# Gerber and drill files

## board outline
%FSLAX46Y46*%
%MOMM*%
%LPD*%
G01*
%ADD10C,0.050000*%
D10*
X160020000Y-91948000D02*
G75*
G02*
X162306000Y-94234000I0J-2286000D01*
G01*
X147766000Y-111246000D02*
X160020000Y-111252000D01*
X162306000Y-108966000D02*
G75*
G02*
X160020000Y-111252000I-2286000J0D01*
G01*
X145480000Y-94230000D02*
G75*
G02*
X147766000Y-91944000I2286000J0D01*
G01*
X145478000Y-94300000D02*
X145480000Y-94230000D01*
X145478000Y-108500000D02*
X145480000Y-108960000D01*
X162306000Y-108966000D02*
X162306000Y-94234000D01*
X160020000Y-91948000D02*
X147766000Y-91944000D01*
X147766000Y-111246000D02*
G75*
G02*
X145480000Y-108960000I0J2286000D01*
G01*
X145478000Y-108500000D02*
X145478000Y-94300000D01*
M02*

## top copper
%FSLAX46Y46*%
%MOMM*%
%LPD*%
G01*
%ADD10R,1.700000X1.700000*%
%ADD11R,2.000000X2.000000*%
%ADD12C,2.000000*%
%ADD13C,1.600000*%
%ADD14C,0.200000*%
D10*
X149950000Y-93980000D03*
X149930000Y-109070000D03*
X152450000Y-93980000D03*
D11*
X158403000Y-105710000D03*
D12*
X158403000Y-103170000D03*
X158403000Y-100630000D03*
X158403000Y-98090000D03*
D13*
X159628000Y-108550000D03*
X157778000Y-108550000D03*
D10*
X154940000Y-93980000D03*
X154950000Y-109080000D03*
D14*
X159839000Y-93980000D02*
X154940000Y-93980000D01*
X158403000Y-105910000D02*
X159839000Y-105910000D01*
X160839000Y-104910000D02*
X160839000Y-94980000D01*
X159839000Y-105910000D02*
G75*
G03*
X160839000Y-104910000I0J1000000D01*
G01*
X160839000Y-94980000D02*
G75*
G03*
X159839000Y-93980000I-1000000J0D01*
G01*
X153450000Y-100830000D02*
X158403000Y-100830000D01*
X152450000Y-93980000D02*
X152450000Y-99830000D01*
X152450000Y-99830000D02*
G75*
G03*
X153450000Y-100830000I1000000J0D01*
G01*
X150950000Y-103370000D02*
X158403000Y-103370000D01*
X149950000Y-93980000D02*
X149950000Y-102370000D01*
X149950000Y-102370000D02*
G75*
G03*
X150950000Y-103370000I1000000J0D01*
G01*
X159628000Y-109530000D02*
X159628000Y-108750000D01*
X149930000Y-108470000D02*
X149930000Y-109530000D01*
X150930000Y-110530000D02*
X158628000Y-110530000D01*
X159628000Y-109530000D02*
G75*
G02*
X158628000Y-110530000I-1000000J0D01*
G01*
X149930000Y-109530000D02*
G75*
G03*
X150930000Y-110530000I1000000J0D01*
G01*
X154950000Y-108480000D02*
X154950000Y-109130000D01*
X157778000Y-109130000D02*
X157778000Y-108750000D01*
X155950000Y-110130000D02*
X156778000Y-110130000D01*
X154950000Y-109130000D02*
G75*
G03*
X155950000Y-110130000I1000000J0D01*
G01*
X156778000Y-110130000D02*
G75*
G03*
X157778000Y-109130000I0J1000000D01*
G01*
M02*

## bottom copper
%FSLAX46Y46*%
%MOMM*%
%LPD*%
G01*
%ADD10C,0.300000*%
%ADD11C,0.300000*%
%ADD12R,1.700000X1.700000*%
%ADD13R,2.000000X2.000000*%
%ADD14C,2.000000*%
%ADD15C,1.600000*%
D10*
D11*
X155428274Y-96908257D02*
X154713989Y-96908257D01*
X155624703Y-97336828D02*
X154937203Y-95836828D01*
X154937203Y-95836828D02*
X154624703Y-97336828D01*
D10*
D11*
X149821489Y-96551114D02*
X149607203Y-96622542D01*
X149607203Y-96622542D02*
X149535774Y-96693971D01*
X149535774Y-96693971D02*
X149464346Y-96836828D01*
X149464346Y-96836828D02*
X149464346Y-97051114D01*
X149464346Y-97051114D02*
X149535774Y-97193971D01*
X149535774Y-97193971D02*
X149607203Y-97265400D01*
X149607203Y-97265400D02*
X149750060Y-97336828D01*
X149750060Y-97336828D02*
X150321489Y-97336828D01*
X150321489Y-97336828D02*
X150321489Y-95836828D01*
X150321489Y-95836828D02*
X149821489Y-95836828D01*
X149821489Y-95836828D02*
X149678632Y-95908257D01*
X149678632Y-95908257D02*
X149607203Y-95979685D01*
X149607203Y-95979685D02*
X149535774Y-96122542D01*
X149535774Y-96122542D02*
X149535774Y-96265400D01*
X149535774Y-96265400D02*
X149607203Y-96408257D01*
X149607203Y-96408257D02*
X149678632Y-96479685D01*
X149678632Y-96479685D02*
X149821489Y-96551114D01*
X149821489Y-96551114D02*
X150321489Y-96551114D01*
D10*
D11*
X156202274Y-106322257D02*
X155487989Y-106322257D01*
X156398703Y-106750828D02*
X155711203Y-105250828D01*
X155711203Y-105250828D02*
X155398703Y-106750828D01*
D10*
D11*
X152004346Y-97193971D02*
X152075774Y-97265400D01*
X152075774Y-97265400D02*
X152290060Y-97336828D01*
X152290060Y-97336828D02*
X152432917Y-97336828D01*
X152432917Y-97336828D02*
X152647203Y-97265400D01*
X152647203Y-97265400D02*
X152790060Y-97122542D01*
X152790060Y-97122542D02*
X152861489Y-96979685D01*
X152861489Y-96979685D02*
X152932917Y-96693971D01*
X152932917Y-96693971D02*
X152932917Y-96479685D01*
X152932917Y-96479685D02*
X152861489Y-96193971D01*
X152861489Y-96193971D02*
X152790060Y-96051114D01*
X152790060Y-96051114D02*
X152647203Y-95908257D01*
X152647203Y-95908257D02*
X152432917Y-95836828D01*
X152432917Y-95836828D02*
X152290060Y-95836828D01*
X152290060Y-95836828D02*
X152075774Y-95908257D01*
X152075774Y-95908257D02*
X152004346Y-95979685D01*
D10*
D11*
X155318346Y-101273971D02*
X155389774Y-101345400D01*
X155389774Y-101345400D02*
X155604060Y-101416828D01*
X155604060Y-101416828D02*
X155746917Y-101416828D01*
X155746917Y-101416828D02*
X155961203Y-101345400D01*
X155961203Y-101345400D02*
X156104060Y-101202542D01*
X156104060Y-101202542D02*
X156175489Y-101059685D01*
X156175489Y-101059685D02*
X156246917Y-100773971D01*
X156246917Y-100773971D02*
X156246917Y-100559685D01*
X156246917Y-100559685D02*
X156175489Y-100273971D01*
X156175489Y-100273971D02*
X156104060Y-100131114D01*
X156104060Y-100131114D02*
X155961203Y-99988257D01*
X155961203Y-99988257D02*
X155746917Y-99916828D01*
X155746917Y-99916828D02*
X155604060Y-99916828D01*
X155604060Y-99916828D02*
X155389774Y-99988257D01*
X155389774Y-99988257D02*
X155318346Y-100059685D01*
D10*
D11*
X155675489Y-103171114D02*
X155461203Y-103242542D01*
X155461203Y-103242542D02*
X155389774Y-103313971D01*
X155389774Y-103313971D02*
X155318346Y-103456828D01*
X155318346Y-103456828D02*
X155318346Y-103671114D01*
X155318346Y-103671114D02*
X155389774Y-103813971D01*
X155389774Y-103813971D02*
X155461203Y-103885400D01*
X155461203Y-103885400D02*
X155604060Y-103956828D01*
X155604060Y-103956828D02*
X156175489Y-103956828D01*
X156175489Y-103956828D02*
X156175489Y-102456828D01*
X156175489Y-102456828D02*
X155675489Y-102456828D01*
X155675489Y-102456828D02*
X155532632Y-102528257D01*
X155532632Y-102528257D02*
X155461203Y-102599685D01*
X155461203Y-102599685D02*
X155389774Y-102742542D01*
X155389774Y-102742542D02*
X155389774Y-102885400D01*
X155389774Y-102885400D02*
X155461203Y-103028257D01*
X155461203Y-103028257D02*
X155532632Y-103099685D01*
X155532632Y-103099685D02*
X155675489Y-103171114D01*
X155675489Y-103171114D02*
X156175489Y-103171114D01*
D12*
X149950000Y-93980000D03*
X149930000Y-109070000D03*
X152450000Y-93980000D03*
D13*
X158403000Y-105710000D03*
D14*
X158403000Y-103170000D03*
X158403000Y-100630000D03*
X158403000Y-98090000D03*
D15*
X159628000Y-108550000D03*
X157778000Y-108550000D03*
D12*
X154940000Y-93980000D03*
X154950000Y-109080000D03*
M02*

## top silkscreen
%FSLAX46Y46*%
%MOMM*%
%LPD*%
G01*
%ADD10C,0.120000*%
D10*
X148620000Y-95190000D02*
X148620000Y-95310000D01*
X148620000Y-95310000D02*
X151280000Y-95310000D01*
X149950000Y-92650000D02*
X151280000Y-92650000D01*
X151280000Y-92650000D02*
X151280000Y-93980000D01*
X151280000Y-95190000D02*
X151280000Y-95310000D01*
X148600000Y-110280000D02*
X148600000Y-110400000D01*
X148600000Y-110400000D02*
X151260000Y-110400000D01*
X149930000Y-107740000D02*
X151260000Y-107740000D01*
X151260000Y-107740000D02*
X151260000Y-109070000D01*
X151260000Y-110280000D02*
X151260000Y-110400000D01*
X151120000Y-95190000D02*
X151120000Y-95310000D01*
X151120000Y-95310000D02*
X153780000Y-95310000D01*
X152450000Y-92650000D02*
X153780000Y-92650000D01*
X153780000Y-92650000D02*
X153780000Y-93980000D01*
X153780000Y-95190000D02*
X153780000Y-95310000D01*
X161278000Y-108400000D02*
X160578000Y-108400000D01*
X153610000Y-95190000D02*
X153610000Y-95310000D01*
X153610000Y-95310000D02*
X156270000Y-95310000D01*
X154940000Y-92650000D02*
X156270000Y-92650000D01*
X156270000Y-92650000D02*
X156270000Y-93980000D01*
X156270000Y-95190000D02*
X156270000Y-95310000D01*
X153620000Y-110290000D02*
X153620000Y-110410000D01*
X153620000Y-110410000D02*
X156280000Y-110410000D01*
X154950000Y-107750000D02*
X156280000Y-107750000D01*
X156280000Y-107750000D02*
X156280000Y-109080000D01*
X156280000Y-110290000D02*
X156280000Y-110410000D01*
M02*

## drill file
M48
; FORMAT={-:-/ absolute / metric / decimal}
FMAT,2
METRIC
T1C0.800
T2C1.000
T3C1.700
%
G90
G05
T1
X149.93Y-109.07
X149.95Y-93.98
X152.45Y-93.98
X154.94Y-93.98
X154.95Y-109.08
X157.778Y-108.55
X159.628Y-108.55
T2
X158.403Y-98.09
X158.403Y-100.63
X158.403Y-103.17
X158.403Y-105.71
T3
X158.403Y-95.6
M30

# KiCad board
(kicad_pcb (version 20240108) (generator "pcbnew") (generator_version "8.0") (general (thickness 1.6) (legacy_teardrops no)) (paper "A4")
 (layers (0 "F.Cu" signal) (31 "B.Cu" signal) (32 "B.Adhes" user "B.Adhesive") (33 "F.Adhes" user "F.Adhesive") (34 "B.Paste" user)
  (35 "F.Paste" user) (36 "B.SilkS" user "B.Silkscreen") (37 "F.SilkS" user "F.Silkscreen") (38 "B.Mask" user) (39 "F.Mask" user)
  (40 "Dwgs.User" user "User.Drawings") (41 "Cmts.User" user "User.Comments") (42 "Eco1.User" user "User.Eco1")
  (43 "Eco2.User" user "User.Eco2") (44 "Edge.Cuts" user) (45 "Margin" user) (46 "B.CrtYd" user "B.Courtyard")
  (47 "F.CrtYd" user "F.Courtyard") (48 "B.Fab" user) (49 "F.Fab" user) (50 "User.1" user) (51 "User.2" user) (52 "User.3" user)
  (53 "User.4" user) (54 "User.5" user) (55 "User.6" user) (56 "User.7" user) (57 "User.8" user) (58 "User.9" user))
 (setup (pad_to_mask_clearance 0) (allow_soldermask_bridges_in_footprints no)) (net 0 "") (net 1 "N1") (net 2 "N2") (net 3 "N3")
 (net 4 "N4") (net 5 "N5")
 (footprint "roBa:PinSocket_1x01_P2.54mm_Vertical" (layer "F.Cu") (at 149.95 93.98)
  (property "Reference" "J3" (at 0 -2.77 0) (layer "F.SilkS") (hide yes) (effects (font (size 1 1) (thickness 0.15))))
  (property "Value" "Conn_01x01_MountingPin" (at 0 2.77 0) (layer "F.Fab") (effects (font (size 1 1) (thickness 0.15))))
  (fp_line (start -1.33 1.21) (end -1.33 1.33) (stroke (width 0.12) (type solid)) (layer "F.SilkS"))
  (fp_line (start -1.33 1.33) (end 1.33 1.33) (stroke (width 0.12) (type solid)) (layer "F.SilkS"))
  (fp_line (start 0 -1.33) (end 1.33 -1.33) (stroke (width 0.12) (type solid)) (layer "F.SilkS"))
  (fp_line (start 1.33 -1.33) (end 1.33 0) (stroke (width 0.12) (type solid)) (layer "F.SilkS"))
  (fp_line (start 1.33 1.21) (end 1.33 1.33) (stroke (width 0.12) (type solid)) (layer "F.SilkS"))
  (pad "1" thru_hole rect (at 0 0) (size 1.7 1.7) (drill 0.8) (layers "*.Cu" "*.Mask") (remove_unused_layers no) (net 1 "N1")))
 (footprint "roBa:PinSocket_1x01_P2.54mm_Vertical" (layer "F.Cu") (at 149.93 109.07)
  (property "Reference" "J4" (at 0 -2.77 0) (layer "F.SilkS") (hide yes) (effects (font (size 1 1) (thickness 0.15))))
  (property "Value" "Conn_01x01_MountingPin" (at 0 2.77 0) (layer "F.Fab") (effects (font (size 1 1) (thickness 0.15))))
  (fp_line (start -1.33 1.21) (end -1.33 1.33) (stroke (width 0.12) (type solid)) (layer "F.SilkS"))
  (fp_line (start -1.33 1.33) (end 1.33 1.33) (stroke (width 0.12) (type solid)) (layer "F.SilkS"))
  (fp_line (start 0 -1.33) (end 1.33 -1.33) (stroke (width 0.12) (type solid)) (layer "F.SilkS"))
  (fp_line (start 1.33 -1.33) (end 1.33 0) (stroke (width 0.12) (type solid)) (layer "F.SilkS"))
  (fp_line (start 1.33 1.21) (end 1.33 1.33) (stroke (width 0.12) (type solid)) (layer "F.SilkS"))
  (pad "1" thru_hole rect (at 0 0) (size 1.7 1.7) (drill 0.8) (layers "*.Cu" "*.Mask") (remove_unused_layers no) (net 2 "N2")))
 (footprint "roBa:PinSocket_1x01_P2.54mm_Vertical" (layer "F.Cu") (at 152.45 93.98)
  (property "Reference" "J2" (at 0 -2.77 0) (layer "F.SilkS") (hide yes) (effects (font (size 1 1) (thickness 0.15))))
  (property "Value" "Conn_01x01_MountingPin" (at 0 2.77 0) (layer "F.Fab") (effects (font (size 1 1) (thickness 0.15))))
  (fp_line (start -1.33 1.21) (end -1.33 1.33) (stroke (width 0.12) (type solid)) (layer "F.SilkS"))
  (fp_line (start -1.33 1.33) (end 1.33 1.33) (stroke (width 0.12) (type solid)) (layer "F.SilkS"))
  (fp_line (start 0 -1.33) (end 1.33 -1.33) (stroke (width 0.12) (type solid)) (layer "F.SilkS"))
  (fp_line (start 1.33 -1.33) (end 1.33 0) (stroke (width 0.12) (type solid)) (layer "F.SilkS"))
  (fp_line (start 1.33 1.21) (end 1.33 1.33) (stroke (width 0.12) (type solid)) (layer "F.SilkS"))
  (pad "1" thru_hole rect (at 0 0) (size 1.7 1.7) (drill 0.8) (layers "*.Cu" "*.Mask") (remove_unused_layers no) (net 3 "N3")))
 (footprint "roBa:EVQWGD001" (layer "F.Cu") (at 151.518 101.4 180)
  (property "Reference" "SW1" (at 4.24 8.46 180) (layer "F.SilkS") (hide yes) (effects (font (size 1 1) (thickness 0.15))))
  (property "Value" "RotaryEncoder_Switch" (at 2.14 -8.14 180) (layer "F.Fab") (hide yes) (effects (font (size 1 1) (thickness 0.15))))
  (fp_line (start -9.76 -7) (end -9.06 -7) (stroke (width 0.12) (type solid)) (layer "F.SilkS"))
  (fp_line (start 6.04 -7.1) (end 6.04 7.1) (stroke (width 0.05) (type solid)) (layer "Edge.Cuts"))
  (pad "" np_thru_hole circle (at -6.885 5.8 180) (size 1.7 1.7) (drill 1.7) (layers "*.Cu" "*.Mask"))
  (pad "A" thru_hole rect (at -6.885 -4.31 180) (size 2 2) (drill 1) (layers "*.Cu" "*.Mask") (remove_unused_layers no) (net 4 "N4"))
  (pad "B" thru_hole circle (at -6.885 -1.77 180) (size 2 2) (drill 1) (layers "*.Cu" "*.Mask") (remove_unused_layers no) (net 1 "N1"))
  (pad "C" thru_hole circle (at -6.885 0.77 180) (size 2 2) (drill 1) (layers "*.Cu" "*.Mask") (remove_unused_layers no) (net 3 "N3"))
  (pad "D" thru_hole circle (at -6.885 3.31 180) (size 2 2) (drill 1) (layers "*.Cu" "*.Mask") (remove_unused_layers no))
  (pad "S1" thru_hole circle (at -8.11 -7.15 180) (size 1.6 1.6) (drill 0.8) (layers "*.Cu" "*.Mask") (remove_unused_layers no) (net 2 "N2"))
  (pad "S2" thru_hole circle (at -6.26 -7.15 180) (size 1.6 1.6) (drill 0.8) (layers "*.Cu" "*.Mask") (remove_unused_layers no) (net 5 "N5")))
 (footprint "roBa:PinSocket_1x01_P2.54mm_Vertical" (layer "F.Cu") (at 154.94 93.98)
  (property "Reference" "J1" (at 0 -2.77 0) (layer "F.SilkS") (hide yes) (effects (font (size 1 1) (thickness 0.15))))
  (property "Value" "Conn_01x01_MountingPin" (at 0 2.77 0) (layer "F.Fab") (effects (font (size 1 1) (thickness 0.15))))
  (fp_line (start -1.33 1.21) (end -1.33 1.33) (stroke (width 0.12) (type solid)) (layer "F.SilkS"))
  (fp_line (start -1.33 1.33) (end 1.33 1.33) (stroke (width 0.12) (type solid)) (layer "F.SilkS"))
  (fp_line (start 0 -1.33) (end 1.33 -1.33) (stroke (width 0.12) (type solid)) (layer "F.SilkS"))
  (fp_line (start 1.33 -1.33) (end 1.33 0) (stroke (width 0.12) (type solid)) (layer "F.SilkS"))
  (fp_line (start 1.33 1.21) (end 1.33 1.33) (stroke (width 0.12) (type solid)) (layer "F.SilkS"))
  (pad "1" thru_hole rect (at 0 0) (size 1.7 1.7) (drill 0.8) (layers "*.Cu" "*.Mask") (remove_unused_layers no) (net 4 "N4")))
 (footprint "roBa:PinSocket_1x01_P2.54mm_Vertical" (layer "F.Cu") (at 154.95 109.08)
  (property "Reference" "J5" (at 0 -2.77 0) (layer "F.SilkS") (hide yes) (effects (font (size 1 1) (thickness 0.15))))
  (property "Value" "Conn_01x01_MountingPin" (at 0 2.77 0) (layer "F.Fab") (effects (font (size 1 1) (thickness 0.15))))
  (fp_line (start -1.33 1.21) (end -1.33 1.33) (stroke (width 0.12) (type solid)) (layer "F.SilkS"))
  (fp_line (start -1.33 1.33) (end 1.33 1.33) (stroke (width 0.12) (type solid)) (layer "F.SilkS"))
  (fp_line (start 0 -1.33) (end 1.33 -1.33) (stroke (width 0.12) (type solid)) (layer "F.SilkS"))
  (fp_line (start 1.33 -1.33) (end 1.33 0) (stroke (width 0.12) (type solid)) (layer "F.SilkS"))
  (fp_line (start 1.33 1.21) (end 1.33 1.33) (stroke (width 0.12) (type solid)) (layer "F.SilkS"))
  (pad "1" thru_hole rect (at 0 0) (size 1.7 1.7) (drill 0.8) (layers "*.Cu" "*.Mask") (remove_unused_layers no) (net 5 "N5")))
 (gr_arc (start 160.02 91.948) (mid 161.636446 92.617554) (end 162.306 94.234) (stroke (width 0.05) (type default)) (layer "Edge.Cuts"))
 (gr_line (start 147.766 111.246) (end 160.02 111.252) (stroke (width 0.05) (type default)) (layer "Edge.Cuts"))
 (gr_arc (start 162.306 108.966) (mid 161.636446 110.582446) (end 160.02 111.252) (stroke (width 0.05) (type default)) (layer "Edge.Cuts"))
 (gr_arc (start 145.48 94.23) (mid 146.149557 92.61357) (end 147.766 91.944) (stroke (width 0.05) (type default)) (layer "Edge.Cuts"))
 (gr_line (start 145.478 94.3) (end 145.48 94.23) (stroke (width 0.05) (type default)) (layer "Edge.Cuts"))
 (gr_line (start 145.478 108.5) (end 145.48 108.96) (stroke (width 0.05) (type default)) (layer "Edge.Cuts"))
 (gr_line (start 162.306 108.966) (end 162.306 94.234) (stroke (width 0.05) (type default)) (layer "Edge.Cuts"))
 (gr_line (start 160.02 91.948) (end 147.766 91.944) (stroke (width 0.05) (type default)) (layer "Edge.Cuts"))
 (gr_arc (start 147.766 111.246) (mid 146.14954 110.57646) (end 145.48 108.96) (stroke (width 0.05) (type default)) (layer "Edge.Cuts"))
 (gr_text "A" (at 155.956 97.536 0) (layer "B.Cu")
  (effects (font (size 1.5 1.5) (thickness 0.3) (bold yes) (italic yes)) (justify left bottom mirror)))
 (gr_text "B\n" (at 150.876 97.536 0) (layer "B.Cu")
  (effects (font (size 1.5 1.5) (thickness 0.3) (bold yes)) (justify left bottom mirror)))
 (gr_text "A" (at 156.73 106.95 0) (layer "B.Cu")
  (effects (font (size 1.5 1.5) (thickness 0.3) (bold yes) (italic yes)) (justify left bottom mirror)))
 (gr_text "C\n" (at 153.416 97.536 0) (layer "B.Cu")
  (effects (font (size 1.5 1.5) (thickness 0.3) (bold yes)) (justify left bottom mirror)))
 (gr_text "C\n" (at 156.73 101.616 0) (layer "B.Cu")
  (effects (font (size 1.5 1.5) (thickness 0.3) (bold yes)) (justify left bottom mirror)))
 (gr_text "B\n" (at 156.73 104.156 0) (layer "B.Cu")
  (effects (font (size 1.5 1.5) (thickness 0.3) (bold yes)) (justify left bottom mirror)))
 (segment (start 159.839 93.98) (end 154.94 93.98) (width 0.2) (layer "F.Cu") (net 4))
 (segment (start 158.403 105.91) (end 159.839 105.91) (width 0.2) (layer "F.Cu") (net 4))
 (segment (start 160.839 104.91) (end 160.839 94.98) (width 0.2) (layer "F.Cu") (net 4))
 (arc (start 159.839 105.91) (mid 160.546107 105.617107) (end 160.839 104.91) (width 0.2) (layer "F.Cu") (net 4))
 (arc (start 160.839 94.98) (mid 160.546107 94.272893) (end 159.839 93.98) (width 0.2) (layer "F.Cu") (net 4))
 (segment (start 153.45 100.83) (end 158.403 100.83) (width 0.2) (layer "F.Cu") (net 3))
 (segment (start 152.45 93.98) (end 152.45 99.83) (width 0.2) (layer "F.Cu") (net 3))
 (arc (start 152.45 99.83) (mid 152.742893 100.537107) (end 153.45 100.83) (width 0.2) (layer "F.Cu") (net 3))
 (segment (start 150.95 103.37) (end 158.403 103.37) (width 0.2) (layer "F.Cu") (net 1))
 (segment (start 149.95 93.98) (end 149.95 102.37) (width 0.2) (layer "F.Cu") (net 1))
 (arc (start 149.95 102.37) (mid 150.242893 103.077107) (end 150.95 103.37) (width 0.2) (layer "F.Cu") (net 1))
 (segment (start 159.628 109.53) (end 159.628 108.75) (width 0.2) (layer "F.Cu") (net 2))
 (segment (start 149.93 108.47) (end 149.93 109.53) (width 0.2) (layer "F.Cu") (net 2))
 (segment (start 150.93 110.53) (end 158.628 110.53) (width 0.2) (layer "F.Cu") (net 2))
 (arc (start 159.628 109.53) (mid 159.335107 110.237107) (end 158.628 110.53) (width 0.2) (layer "F.Cu") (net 2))
 (arc (start 149.93 109.53) (mid 150.222893 110.237107) (end 150.93 110.53) (width 0.2) (layer "F.Cu") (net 2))
 (segment (start 154.95 108.48) (end 154.95 109.13) (width 0.2) (layer "F.Cu") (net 5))
 (segment (start 157.778 109.13) (end 157.778 108.75) (width 0.2) (layer "F.Cu") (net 5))
 (segment (start 155.95 110.13) (end 156.778 110.13) (width 0.2) (layer "F.Cu") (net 5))
 (arc (start 154.95 109.13) (mid 155.242893 109.837107) (end 155.95 110.13) (width 0.2) (layer "F.Cu") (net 5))
 (arc (start 156.778 110.13) (mid 157.485107 109.837107) (end 157.778 109.13) (width 0.2) (layer "F.Cu") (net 5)))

